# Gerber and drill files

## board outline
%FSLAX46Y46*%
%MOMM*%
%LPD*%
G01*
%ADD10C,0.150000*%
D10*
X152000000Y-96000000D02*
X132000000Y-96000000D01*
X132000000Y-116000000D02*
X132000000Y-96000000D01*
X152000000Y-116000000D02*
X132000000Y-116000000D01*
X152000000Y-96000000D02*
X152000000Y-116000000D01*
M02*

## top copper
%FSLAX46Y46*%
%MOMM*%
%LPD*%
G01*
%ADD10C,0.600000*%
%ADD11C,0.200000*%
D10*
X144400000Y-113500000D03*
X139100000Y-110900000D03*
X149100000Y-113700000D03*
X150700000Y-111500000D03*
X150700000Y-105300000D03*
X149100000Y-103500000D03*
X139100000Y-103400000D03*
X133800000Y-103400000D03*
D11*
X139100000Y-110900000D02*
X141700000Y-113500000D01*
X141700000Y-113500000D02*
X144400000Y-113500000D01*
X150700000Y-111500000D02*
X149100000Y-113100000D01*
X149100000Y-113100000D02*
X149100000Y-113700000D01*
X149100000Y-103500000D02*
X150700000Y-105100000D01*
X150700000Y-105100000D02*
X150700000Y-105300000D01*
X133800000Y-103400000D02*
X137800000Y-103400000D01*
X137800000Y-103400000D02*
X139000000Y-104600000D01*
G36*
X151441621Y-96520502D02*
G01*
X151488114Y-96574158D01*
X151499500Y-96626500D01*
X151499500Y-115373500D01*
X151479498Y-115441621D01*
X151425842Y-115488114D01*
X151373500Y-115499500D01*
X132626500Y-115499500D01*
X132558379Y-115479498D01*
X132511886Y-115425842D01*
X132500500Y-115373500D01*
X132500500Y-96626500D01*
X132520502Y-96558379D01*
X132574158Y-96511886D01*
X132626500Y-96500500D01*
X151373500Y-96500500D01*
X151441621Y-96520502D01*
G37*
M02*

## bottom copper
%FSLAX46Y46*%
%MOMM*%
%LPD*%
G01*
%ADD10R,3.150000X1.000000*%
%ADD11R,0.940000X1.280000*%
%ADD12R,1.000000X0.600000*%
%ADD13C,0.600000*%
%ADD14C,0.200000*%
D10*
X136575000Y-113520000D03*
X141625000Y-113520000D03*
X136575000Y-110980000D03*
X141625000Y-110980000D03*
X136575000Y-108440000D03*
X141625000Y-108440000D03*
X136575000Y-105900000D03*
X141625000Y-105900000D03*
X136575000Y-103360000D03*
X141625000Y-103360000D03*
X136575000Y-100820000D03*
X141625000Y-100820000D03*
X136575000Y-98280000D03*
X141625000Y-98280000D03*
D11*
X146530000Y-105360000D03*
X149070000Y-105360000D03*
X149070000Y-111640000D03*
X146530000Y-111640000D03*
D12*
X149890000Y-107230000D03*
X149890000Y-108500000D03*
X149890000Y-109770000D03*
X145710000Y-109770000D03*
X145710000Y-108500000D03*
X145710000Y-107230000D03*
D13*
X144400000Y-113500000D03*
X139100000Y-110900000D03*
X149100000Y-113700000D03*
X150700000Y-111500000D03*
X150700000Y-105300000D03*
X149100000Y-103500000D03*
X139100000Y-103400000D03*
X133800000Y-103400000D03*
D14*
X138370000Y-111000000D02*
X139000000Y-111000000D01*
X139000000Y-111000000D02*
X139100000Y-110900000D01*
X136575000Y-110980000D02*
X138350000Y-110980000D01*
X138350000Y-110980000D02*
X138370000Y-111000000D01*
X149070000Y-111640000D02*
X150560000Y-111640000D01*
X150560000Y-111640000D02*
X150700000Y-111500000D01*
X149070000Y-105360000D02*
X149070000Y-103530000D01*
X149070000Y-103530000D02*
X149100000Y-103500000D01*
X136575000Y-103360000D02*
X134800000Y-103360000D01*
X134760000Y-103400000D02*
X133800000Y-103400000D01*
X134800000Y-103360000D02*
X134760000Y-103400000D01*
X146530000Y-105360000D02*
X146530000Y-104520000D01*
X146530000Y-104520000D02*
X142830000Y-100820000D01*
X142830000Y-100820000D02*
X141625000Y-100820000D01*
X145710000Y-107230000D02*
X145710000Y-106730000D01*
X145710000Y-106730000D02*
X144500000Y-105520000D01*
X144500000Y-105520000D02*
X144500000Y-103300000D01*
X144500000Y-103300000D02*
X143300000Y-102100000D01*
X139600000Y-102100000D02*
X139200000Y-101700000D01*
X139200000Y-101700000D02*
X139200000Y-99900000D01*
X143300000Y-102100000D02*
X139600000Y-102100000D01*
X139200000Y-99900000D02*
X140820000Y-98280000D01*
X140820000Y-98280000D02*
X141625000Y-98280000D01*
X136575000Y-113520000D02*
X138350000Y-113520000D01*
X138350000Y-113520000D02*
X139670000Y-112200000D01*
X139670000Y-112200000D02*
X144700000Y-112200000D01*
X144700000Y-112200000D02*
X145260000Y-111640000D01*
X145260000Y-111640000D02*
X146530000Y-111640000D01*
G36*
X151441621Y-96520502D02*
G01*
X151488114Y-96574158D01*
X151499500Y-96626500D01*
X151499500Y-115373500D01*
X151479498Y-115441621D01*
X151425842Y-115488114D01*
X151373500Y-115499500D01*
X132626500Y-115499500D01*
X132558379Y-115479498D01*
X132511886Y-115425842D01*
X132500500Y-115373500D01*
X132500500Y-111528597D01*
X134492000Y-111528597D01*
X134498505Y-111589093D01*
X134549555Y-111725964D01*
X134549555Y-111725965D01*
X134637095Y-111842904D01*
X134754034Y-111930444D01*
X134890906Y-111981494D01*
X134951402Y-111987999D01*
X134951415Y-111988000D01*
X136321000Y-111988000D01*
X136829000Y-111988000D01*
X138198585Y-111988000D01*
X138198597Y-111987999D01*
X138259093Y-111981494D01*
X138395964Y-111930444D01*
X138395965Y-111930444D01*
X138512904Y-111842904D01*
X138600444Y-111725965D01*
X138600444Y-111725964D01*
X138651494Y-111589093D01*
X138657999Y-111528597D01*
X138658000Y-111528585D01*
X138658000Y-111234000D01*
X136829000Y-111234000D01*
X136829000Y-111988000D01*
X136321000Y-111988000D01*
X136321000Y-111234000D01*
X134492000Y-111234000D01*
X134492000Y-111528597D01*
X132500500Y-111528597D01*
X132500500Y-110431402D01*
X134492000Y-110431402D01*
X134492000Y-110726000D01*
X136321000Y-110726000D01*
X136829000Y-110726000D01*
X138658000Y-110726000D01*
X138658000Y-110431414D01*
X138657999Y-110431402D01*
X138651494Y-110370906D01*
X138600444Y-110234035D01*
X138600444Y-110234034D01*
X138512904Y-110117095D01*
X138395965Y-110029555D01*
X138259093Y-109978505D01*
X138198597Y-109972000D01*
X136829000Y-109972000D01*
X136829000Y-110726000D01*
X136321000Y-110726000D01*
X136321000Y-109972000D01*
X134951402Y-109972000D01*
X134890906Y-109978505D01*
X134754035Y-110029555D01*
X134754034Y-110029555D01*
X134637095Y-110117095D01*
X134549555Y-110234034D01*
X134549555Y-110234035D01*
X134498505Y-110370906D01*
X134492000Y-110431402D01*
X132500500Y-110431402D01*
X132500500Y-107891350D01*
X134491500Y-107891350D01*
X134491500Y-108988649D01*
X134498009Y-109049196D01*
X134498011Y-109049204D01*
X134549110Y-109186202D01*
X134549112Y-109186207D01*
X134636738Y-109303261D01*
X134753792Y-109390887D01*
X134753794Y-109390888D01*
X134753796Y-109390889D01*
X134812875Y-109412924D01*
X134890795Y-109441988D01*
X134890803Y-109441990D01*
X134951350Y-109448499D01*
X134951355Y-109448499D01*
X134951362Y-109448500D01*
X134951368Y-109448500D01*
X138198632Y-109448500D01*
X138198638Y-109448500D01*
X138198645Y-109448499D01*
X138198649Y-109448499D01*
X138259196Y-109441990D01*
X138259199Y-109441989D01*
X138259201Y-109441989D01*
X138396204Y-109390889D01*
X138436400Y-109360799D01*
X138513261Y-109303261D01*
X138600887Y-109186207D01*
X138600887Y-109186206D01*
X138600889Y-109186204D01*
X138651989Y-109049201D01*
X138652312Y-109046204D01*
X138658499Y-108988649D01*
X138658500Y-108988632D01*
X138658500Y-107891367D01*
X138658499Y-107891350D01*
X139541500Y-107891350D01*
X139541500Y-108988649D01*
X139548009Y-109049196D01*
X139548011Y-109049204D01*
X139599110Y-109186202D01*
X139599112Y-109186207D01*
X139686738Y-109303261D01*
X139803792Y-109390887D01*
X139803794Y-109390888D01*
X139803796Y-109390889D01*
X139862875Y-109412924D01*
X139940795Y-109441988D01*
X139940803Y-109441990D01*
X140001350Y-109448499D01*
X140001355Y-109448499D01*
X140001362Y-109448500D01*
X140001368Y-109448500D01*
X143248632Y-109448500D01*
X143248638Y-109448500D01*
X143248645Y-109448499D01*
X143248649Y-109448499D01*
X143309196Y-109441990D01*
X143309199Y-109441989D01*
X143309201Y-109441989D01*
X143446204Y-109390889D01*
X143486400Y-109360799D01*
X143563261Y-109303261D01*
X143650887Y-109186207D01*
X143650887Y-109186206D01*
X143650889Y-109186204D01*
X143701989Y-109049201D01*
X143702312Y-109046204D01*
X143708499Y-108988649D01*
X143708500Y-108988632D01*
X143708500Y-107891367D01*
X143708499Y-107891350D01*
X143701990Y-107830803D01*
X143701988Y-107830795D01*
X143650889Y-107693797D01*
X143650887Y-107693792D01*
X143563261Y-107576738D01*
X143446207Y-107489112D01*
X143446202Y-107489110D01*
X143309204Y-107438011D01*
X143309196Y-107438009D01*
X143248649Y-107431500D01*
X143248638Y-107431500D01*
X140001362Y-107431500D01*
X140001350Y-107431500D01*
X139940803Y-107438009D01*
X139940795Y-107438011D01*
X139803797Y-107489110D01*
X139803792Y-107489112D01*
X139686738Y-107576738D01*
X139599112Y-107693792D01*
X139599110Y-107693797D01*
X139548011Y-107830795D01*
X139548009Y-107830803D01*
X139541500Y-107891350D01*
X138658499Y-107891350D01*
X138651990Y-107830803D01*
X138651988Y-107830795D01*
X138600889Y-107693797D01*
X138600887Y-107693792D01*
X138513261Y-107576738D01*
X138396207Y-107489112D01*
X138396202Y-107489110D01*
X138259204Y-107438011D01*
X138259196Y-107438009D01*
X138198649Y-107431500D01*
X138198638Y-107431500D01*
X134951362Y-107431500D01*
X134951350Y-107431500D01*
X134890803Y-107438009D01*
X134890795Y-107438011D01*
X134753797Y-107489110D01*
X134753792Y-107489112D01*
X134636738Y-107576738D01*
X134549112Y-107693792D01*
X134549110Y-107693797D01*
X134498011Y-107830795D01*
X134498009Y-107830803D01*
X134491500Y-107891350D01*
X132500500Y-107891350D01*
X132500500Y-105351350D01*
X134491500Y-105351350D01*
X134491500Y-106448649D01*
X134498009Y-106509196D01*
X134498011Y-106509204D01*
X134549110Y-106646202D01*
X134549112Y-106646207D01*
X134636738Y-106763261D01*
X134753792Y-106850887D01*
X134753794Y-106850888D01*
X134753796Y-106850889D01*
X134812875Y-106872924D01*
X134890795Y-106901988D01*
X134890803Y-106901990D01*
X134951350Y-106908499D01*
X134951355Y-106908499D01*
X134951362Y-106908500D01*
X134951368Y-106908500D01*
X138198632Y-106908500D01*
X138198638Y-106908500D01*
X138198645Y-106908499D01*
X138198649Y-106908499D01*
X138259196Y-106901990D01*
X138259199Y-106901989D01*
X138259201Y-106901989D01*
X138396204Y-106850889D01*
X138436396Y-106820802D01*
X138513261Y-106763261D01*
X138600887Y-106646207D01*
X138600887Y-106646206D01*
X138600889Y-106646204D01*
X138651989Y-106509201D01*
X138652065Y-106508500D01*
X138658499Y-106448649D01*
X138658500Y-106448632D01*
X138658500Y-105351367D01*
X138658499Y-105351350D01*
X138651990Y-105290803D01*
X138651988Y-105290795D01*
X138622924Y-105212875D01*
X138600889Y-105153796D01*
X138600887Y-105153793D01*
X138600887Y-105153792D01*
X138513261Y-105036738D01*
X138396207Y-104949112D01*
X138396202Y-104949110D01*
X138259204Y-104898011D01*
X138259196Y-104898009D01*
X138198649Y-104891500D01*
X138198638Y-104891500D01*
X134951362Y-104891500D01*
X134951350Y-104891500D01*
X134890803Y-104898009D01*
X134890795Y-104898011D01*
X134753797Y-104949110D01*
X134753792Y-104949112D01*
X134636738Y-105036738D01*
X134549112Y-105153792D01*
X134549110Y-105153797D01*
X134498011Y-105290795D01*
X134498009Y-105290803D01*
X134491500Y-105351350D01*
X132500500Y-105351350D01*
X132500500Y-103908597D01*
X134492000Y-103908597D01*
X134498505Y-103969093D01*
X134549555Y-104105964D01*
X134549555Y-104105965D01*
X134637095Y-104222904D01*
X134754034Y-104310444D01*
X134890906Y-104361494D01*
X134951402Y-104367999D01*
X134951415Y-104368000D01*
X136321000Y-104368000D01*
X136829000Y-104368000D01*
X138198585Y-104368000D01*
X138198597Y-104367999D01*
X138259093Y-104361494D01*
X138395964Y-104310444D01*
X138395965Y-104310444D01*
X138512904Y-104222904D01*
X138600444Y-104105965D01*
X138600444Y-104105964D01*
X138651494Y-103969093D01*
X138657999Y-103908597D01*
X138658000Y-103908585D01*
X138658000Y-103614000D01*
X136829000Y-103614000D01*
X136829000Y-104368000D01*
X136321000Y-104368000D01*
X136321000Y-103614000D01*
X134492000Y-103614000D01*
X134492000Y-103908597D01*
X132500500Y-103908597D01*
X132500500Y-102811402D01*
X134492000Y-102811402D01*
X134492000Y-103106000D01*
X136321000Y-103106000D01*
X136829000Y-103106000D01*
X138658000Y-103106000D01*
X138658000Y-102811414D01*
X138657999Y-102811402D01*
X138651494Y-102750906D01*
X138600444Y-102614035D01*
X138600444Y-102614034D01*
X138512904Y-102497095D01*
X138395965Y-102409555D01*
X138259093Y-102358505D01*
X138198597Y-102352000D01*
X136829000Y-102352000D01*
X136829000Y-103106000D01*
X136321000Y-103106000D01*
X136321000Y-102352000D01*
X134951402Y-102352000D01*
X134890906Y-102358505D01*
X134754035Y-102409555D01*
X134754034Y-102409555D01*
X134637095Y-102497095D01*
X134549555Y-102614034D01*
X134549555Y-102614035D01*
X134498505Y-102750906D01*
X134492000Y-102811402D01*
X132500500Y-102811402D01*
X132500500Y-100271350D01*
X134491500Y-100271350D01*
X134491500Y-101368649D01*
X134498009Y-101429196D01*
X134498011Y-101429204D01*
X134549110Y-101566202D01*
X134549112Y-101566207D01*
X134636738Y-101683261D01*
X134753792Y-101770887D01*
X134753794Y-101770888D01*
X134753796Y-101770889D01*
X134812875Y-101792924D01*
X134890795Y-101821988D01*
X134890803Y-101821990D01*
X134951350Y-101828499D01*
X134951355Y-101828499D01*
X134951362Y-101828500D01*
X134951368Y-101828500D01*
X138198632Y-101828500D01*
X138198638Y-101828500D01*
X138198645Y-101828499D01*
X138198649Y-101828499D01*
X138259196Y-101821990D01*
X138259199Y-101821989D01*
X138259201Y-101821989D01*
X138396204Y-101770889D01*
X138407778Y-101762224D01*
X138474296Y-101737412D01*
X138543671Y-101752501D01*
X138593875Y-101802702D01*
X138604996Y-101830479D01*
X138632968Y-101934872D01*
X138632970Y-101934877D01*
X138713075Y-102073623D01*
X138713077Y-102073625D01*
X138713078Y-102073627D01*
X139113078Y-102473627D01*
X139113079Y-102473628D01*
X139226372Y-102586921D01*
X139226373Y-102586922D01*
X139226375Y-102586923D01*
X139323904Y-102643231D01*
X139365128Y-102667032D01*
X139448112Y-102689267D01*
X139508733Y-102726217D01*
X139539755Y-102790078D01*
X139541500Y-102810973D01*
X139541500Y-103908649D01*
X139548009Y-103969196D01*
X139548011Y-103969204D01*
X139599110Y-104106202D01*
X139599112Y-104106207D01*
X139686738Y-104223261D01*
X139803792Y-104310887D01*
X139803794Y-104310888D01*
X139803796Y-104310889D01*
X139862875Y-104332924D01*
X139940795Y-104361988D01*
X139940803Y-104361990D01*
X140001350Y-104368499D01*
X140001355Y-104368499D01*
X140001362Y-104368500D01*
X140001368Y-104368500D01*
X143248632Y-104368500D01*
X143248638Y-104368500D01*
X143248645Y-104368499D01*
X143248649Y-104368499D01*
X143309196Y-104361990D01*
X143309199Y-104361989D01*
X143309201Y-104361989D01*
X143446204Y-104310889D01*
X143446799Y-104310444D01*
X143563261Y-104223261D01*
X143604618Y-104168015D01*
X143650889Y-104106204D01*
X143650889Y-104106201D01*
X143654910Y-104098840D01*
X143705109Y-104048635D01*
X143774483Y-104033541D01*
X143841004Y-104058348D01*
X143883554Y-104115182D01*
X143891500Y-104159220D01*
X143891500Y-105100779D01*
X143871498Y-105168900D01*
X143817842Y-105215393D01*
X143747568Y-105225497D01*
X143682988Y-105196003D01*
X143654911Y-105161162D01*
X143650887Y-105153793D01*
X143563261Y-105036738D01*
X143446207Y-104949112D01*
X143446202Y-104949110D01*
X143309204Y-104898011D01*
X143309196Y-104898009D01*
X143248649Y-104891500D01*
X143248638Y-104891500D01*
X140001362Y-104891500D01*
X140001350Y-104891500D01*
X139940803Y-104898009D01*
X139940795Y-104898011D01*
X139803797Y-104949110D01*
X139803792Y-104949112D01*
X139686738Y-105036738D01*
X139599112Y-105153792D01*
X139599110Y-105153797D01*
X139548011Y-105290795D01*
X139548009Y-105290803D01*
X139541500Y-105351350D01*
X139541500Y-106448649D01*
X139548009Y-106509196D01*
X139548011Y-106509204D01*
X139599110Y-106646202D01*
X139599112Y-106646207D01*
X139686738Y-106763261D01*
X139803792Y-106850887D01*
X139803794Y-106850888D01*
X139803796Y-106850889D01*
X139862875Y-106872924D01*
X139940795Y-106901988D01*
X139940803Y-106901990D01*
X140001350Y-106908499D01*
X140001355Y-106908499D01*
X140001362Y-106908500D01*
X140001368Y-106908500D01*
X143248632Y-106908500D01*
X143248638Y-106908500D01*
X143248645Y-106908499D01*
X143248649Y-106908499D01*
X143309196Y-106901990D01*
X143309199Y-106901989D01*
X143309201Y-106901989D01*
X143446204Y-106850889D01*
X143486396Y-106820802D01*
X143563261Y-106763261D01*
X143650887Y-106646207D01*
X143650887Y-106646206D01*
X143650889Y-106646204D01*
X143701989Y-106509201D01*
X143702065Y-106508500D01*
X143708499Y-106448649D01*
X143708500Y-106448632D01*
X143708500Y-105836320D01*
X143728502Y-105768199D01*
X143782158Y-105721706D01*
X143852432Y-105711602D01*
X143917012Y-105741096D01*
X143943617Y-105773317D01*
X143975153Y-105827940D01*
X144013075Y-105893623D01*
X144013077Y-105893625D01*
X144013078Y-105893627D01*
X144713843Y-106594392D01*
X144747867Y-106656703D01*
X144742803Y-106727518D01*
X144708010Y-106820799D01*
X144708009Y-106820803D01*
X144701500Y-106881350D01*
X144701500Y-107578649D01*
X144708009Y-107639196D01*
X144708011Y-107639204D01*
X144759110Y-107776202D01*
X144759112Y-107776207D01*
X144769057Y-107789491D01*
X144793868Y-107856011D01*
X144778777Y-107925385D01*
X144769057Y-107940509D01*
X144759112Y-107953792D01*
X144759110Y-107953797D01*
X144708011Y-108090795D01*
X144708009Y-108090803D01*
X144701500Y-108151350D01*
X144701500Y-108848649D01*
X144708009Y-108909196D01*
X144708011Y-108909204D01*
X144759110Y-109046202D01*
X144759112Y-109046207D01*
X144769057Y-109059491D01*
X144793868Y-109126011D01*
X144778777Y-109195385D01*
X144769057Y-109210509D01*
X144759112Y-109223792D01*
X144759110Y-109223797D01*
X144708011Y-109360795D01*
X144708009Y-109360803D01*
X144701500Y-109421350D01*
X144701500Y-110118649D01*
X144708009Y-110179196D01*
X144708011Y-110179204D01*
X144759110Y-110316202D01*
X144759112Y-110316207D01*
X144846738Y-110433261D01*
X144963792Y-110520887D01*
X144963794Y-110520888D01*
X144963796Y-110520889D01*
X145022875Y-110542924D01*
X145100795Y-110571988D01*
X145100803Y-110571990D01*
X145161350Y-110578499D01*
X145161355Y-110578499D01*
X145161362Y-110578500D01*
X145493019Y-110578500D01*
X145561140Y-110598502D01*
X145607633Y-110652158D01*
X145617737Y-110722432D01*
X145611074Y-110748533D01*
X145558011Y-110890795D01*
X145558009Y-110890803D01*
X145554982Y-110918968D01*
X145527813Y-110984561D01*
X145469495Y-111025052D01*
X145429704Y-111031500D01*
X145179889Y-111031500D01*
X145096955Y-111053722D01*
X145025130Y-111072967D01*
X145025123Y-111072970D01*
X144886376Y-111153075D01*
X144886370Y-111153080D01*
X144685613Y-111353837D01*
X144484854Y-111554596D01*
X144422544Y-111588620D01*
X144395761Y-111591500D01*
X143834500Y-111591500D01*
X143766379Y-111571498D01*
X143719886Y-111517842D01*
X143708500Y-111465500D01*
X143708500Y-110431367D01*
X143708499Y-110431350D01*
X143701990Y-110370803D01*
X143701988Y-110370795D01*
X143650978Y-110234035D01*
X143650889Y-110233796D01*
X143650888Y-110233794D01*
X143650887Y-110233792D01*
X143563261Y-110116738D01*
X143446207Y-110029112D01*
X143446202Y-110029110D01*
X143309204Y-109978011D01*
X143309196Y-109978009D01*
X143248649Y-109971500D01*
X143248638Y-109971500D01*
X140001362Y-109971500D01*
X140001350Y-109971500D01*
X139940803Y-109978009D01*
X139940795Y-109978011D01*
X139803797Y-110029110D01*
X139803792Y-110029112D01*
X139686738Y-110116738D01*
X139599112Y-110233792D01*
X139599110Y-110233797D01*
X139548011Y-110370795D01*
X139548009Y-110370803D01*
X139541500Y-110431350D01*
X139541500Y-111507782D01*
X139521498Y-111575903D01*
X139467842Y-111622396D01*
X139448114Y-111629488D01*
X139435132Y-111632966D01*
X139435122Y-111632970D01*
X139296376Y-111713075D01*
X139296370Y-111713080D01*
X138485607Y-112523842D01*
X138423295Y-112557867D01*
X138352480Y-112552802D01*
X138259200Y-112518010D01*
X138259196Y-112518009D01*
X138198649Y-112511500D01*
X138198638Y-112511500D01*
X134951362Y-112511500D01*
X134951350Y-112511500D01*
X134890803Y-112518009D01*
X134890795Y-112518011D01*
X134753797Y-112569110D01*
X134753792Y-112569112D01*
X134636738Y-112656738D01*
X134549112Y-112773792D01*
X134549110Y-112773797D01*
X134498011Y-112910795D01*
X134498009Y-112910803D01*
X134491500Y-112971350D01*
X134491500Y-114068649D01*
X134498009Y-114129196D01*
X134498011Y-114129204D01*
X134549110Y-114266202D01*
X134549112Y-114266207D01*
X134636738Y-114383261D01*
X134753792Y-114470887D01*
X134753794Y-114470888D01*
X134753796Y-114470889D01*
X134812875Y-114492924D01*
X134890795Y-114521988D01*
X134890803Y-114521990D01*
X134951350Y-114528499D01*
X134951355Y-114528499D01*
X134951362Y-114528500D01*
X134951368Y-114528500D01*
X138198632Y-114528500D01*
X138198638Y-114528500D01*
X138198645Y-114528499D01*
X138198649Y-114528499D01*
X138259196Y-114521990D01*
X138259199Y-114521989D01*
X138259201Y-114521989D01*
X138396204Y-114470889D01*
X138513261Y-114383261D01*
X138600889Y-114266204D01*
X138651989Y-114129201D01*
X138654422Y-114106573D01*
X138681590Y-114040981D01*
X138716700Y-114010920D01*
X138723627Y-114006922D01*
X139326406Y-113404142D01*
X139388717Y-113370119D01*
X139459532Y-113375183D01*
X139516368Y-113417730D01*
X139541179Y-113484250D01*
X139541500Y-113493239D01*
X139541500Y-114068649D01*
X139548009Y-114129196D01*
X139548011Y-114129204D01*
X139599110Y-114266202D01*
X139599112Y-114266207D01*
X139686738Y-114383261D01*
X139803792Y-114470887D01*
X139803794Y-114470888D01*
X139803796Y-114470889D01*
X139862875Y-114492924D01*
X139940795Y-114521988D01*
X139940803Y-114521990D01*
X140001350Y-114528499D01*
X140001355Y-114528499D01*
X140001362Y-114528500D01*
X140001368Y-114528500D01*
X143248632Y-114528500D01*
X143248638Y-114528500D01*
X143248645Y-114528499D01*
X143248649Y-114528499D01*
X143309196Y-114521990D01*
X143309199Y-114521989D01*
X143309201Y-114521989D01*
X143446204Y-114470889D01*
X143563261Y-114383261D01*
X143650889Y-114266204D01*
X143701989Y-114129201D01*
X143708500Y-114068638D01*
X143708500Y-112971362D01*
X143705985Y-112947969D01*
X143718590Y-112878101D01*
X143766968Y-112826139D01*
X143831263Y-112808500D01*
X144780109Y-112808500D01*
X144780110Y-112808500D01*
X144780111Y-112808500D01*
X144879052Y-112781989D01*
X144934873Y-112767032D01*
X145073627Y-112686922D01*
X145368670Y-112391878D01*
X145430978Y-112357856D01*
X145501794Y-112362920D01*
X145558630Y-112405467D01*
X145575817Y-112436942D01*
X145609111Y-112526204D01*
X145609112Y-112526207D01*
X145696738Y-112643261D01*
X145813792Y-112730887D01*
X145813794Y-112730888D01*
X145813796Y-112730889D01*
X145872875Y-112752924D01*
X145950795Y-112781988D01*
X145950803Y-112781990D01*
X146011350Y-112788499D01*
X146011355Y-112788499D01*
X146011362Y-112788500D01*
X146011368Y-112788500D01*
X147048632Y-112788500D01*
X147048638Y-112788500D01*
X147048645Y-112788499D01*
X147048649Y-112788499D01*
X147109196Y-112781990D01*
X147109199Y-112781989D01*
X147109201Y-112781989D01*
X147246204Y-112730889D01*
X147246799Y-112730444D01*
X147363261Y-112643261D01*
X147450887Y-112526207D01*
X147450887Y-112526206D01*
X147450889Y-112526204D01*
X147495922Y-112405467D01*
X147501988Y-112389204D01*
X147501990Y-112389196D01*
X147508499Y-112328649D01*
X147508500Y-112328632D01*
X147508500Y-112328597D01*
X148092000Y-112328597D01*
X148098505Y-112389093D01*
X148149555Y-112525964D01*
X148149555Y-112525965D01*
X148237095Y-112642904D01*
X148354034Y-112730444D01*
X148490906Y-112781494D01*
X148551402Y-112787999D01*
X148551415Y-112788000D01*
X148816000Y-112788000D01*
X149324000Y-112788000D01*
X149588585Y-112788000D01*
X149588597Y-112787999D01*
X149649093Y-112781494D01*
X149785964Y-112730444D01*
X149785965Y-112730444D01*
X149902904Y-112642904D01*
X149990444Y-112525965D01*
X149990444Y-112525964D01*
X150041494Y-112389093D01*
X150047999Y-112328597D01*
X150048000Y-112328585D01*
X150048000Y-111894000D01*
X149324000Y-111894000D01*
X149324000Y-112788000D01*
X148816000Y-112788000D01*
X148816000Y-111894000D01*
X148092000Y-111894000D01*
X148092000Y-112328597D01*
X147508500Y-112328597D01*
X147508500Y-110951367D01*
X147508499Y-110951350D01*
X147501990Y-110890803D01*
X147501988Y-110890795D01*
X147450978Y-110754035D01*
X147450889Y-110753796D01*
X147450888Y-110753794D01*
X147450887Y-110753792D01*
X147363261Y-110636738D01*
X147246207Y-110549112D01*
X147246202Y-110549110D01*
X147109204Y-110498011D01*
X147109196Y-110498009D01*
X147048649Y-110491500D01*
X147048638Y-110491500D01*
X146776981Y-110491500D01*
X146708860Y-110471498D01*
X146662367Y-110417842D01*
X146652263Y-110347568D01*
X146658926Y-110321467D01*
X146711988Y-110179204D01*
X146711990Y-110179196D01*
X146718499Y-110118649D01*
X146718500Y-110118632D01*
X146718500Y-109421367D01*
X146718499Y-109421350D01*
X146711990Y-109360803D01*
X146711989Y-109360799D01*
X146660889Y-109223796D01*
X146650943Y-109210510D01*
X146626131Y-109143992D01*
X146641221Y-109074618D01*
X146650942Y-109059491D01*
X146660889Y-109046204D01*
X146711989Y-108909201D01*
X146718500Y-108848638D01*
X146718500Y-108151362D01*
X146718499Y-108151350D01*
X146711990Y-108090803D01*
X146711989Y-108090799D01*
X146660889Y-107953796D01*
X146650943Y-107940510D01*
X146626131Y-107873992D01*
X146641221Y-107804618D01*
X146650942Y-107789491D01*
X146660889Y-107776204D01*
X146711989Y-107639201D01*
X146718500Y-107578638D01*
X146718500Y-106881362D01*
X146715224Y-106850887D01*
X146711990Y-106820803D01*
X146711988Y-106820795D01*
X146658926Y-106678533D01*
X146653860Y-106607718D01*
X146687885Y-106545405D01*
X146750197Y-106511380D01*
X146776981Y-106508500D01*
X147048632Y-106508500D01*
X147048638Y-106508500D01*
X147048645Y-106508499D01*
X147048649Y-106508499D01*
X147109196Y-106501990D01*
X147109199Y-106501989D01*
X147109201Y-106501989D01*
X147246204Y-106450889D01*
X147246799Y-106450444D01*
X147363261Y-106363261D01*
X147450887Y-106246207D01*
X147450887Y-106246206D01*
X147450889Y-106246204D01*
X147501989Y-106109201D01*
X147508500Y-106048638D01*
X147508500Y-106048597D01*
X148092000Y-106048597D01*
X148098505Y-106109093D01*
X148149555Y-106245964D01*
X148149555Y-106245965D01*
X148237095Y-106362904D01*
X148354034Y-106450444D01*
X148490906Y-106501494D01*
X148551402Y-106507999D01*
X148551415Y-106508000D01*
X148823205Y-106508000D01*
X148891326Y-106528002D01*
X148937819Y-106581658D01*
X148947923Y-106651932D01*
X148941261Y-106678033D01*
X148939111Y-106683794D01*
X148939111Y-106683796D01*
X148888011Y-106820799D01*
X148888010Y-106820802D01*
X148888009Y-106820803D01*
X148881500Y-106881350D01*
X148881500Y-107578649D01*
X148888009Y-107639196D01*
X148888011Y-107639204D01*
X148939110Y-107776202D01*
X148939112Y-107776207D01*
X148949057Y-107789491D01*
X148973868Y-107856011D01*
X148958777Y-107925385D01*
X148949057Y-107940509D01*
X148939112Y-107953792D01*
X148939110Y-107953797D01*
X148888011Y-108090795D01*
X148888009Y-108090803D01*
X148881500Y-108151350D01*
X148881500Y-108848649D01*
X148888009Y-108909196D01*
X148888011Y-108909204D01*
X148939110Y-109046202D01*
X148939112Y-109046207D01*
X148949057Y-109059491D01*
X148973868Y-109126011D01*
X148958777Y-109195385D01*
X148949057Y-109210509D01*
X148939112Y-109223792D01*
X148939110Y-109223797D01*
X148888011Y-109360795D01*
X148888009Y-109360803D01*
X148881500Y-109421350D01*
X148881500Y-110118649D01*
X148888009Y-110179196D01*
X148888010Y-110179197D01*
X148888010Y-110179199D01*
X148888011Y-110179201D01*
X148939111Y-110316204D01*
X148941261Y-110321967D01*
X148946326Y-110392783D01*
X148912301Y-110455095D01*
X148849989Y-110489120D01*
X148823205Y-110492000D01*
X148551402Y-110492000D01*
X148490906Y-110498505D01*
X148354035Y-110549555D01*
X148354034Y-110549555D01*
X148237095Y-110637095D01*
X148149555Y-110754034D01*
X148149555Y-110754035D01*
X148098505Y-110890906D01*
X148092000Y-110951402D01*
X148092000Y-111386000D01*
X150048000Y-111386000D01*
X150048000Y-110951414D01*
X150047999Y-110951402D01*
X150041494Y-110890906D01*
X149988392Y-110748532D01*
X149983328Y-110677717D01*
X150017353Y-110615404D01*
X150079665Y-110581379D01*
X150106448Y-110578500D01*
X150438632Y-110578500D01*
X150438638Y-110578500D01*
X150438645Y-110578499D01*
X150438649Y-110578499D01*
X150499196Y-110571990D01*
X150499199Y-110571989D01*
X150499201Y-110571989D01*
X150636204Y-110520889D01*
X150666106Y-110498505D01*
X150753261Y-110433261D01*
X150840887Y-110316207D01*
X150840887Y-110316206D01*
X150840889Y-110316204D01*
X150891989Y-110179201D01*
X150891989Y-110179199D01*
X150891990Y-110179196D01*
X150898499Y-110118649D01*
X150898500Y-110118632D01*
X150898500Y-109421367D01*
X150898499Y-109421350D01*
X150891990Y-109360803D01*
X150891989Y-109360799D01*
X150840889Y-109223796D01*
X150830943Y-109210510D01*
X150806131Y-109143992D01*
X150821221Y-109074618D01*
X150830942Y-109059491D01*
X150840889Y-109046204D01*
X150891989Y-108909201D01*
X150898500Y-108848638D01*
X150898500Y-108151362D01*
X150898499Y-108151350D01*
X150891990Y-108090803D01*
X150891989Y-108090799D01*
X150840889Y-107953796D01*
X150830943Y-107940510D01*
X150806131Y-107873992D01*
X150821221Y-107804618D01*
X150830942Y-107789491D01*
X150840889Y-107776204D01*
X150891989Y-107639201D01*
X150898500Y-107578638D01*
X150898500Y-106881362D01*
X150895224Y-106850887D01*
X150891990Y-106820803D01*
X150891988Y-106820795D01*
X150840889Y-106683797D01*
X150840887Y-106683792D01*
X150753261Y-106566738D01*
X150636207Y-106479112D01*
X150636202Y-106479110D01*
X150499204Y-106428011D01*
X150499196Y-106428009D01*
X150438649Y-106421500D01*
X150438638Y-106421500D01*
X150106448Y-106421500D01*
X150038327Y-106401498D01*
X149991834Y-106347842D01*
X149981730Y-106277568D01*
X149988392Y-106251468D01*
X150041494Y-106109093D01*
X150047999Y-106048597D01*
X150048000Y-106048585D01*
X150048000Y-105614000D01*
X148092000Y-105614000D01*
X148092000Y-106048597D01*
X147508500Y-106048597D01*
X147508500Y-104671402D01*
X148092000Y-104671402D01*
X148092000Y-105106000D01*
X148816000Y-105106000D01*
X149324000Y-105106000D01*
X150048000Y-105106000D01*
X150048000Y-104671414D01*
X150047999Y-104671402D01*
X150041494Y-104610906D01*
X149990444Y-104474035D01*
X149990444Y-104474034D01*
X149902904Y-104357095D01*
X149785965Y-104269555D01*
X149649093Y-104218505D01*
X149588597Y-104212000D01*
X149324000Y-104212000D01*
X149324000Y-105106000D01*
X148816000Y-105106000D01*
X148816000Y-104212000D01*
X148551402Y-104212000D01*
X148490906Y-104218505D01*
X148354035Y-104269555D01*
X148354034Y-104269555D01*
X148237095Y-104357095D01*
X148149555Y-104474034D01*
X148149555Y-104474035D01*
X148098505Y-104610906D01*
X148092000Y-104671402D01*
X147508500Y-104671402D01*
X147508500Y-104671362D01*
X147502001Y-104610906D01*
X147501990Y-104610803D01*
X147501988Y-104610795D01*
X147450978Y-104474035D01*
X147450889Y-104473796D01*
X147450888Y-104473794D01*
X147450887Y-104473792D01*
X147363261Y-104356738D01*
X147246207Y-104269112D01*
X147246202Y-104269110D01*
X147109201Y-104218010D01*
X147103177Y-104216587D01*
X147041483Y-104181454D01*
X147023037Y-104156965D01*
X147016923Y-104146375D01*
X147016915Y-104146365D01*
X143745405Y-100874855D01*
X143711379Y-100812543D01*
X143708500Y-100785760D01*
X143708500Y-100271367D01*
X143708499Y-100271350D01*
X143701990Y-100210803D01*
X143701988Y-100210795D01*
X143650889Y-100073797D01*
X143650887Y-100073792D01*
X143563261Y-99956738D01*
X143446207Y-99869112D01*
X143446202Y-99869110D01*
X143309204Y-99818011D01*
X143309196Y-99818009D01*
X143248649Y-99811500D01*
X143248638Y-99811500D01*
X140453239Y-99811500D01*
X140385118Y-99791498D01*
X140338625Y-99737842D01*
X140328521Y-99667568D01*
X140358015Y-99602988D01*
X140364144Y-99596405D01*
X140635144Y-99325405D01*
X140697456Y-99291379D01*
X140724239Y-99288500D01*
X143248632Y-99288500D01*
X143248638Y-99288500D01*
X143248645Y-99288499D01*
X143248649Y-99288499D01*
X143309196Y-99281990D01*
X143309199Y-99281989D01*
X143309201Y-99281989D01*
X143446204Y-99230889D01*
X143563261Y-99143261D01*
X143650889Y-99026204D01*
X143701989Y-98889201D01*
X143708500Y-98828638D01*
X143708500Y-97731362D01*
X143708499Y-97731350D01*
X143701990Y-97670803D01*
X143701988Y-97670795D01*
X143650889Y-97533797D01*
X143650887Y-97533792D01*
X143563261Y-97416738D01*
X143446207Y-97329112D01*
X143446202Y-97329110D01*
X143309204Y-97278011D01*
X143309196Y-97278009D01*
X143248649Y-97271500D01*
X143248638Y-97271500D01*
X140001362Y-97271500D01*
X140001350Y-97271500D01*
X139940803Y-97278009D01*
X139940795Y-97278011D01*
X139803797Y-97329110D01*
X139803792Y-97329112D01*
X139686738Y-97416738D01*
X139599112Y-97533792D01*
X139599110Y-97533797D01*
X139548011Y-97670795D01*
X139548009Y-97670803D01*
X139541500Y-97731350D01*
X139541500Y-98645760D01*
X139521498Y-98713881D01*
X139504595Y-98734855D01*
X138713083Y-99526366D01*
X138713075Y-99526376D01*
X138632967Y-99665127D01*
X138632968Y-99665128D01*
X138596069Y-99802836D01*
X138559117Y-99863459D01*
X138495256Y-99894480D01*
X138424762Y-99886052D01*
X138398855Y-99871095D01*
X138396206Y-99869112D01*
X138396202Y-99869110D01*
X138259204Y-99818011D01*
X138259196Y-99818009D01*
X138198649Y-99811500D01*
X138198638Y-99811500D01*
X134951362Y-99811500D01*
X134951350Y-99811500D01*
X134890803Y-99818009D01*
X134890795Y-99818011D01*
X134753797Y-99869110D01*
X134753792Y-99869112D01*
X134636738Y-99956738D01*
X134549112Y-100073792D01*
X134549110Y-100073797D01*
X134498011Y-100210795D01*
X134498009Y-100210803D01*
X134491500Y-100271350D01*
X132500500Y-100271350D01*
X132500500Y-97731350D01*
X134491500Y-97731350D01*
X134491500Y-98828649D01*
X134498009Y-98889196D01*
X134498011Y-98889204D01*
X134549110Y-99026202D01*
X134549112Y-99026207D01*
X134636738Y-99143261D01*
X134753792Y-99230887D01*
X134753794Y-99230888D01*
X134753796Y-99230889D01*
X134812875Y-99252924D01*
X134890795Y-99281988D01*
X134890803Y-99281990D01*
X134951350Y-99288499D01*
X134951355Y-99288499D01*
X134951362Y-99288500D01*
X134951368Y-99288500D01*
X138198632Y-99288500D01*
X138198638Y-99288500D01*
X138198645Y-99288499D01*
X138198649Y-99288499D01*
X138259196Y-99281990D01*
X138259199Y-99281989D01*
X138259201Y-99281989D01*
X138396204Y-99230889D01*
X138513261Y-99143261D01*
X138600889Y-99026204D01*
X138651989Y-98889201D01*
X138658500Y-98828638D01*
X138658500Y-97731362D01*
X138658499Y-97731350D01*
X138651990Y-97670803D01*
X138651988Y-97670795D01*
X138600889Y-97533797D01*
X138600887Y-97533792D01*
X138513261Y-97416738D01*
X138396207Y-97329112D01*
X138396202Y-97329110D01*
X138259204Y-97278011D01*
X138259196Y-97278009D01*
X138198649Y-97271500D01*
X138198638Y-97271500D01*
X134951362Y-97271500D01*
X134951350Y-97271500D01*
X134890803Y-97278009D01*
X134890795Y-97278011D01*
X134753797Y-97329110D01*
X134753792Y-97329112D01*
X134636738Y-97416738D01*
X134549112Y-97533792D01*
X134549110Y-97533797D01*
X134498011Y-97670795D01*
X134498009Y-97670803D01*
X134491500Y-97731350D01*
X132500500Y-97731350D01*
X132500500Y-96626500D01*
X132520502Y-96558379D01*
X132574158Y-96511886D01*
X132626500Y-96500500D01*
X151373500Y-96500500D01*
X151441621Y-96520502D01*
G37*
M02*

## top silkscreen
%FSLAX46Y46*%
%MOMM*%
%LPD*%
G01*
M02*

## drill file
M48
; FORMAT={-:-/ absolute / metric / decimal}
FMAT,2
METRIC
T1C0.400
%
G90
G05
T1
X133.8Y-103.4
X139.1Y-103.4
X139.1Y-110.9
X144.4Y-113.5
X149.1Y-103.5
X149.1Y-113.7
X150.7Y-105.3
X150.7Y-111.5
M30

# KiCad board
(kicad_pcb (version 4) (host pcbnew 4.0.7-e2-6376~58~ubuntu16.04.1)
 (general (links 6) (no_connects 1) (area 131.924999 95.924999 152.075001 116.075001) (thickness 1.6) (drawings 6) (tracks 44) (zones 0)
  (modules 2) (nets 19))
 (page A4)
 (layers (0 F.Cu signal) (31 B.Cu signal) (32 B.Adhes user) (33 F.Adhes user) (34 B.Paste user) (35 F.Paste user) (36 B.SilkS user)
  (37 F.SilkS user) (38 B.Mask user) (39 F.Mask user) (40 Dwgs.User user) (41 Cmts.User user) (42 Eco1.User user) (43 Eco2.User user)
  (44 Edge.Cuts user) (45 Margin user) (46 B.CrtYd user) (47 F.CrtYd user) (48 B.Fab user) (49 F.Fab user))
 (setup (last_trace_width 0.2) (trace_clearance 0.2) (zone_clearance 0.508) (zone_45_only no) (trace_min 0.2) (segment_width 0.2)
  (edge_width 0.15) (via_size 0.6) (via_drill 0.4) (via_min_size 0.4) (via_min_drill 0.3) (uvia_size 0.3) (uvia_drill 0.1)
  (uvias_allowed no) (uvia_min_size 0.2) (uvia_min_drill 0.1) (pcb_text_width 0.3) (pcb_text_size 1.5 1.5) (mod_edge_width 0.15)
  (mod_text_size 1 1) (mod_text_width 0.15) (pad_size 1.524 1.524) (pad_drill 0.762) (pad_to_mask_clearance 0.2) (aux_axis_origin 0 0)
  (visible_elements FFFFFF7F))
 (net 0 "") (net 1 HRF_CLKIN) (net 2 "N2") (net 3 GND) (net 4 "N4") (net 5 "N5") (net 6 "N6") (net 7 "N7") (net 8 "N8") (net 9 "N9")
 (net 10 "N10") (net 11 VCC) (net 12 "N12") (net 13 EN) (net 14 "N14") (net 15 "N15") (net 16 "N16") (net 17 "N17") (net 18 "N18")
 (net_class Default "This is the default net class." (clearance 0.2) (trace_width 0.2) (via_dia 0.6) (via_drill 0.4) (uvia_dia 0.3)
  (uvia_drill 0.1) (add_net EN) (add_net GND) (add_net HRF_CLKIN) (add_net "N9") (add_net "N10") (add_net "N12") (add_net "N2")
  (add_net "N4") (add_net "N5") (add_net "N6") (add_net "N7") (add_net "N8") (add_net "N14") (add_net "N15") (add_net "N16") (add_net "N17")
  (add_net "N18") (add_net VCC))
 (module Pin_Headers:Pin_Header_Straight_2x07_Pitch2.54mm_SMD (layer B.Cu) (at 139.1 105.9)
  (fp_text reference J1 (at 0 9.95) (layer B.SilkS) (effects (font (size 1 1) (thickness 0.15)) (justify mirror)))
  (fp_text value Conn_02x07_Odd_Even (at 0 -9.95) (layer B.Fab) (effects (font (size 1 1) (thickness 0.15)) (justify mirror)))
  (pad 1 smd rect (at -2.525 7.62) (size 3.15 1) (layers B.Cu B.Paste B.Mask) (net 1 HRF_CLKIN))
  (pad 2 smd rect (at 2.525 7.62) (size 3.15 1) (layers B.Cu B.Paste B.Mask) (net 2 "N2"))
  (pad 3 smd rect (at -2.525 5.08) (size 3.15 1) (layers B.Cu B.Paste B.Mask) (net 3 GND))
  (pad 4 smd rect (at 2.525 5.08) (size 3.15 1) (layers B.Cu B.Paste B.Mask) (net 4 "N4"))
  (pad 5 smd rect (at -2.525 2.54) (size 3.15 1) (layers B.Cu B.Paste B.Mask) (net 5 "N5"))
  (pad 6 smd rect (at 2.525 2.54) (size 3.15 1) (layers B.Cu B.Paste B.Mask) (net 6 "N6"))
  (pad 7 smd rect (at -2.525 0) (size 3.15 1) (layers B.Cu B.Paste B.Mask) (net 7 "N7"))
  (pad 8 smd rect (at 2.525 0) (size 3.15 1) (layers B.Cu B.Paste B.Mask) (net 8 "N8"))
  (pad 9 smd rect (at -2.525 -2.54) (size 3.15 1) (layers B.Cu B.Paste B.Mask) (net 3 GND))
  (pad 10 smd rect (at 2.525 -2.54) (size 3.15 1) (layers B.Cu B.Paste B.Mask) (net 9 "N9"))
  (pad 11 smd rect (at -2.525 -5.08) (size 3.15 1) (layers B.Cu B.Paste B.Mask) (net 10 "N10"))
  (pad 12 smd rect (at 2.525 -5.08) (size 3.15 1) (layers B.Cu B.Paste B.Mask) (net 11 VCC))
  (pad 13 smd rect (at -2.525 -7.62) (size 3.15 1) (layers B.Cu B.Paste B.Mask) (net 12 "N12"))
  (pad 14 smd rect (at 2.525 -7.62) (size 3.15 1) (layers B.Cu B.Paste B.Mask) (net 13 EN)))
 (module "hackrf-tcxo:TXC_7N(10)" (layer B.Cu) (at 147.8 108.5 270)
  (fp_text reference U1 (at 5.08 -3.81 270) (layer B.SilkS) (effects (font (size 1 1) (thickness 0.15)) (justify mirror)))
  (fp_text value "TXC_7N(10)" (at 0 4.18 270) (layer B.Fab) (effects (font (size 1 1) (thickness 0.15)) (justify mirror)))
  (pad 9 smd rect (at -3.14 1.27 270) (size 1.28 0.94) (layers B.Cu B.Paste B.Mask) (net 11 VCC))
  (pad 10 smd rect (at -3.14 -1.27 270) (size 1.28 0.94) (layers B.Cu B.Paste B.Mask) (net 3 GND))
  (pad 4 smd rect (at 3.14 -1.27 270) (size 1.28 0.94) (layers B.Cu B.Paste B.Mask) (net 3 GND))
  (pad 5 smd rect (at 3.14 1.27 270) (size 1.28 0.94) (layers B.Cu B.Paste B.Mask) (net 1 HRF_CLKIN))
  (pad 1 smd rect (at -1.27 -2.09 270) (size 0.6 1) (layers B.Cu B.Paste B.Mask) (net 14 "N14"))
  (pad 2 smd rect (at 0 -2.09 270) (size 0.6 1) (layers B.Cu B.Paste B.Mask) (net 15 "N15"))
  (pad 3 smd rect (at 1.27 -2.09 270) (size 0.6 1) (layers B.Cu B.Paste B.Mask) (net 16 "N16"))
  (pad 6 smd rect (at 1.27 2.09 270) (size 0.6 1) (layers B.Cu B.Paste B.Mask) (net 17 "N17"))
  (pad 7 smd rect (at 0 2.09 270) (size 0.6 1) (layers B.Cu B.Paste B.Mask) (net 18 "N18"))
  (pad 8 smd rect (at -1.27 2.09 270) (size 0.6 1) (layers B.Cu B.Paste B.Mask) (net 13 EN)))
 (gr_line (start 152 96) (end 132 96) (angle 90) (layer Edge.Cuts) (width 0.15))
 (gr_line (start 132 116) (end 132 96) (angle 90) (layer Edge.Cuts) (width 0.15))
 (gr_line (start 152 116) (end 132 116) (angle 90) (layer Edge.Cuts) (width 0.15))
 (gr_line (start 152 96) (end 152 116) (angle 90) (layer Edge.Cuts) (width 0.15))
 (segment (start 139.1 110.9) (end 141.7 113.5) (width 0.2) (layer F.Cu) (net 3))
 (segment (start 141.7 113.5) (end 144.4 113.5) (width 0.2) (layer F.Cu) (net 3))
 (via (at 144.4 113.5) (size 0.6) (drill 0.4) (layers F.Cu B.Cu) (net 3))
 (segment (start 138.37 111) (end 139 111) (width 0.2) (layer B.Cu) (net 3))
 (segment (start 139 111) (end 139.1 110.9) (width 0.2) (layer B.Cu) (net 3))
 (via (at 139.1 110.9) (size 0.6) (drill 0.4) (layers F.Cu B.Cu) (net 3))
 (segment (start 136.575 110.98) (end 138.35 110.98) (width 0.2) (layer B.Cu) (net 3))
 (segment (start 138.35 110.98) (end 138.37 111) (width 0.2) (layer B.Cu) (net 3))
 (segment (start 150.7 111.5) (end 149.1 113.1) (width 0.2) (layer F.Cu) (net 3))
 (segment (start 149.1 113.1) (end 149.1 113.7) (width 0.2) (layer F.Cu) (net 3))
 (via (at 149.1 113.7) (size 0.6) (drill 0.4) (layers F.Cu B.Cu) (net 3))
 (segment (start 149.07 111.64) (end 150.56 111.64) (width 0.2) (layer B.Cu) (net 3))
 (segment (start 150.56 111.64) (end 150.7 111.5) (width 0.2) (layer B.Cu) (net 3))
 (via (at 150.7 111.5) (size 0.6) (drill 0.4) (layers F.Cu B.Cu) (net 3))
 (segment (start 149.1 103.5) (end 150.7 105.1) (width 0.2) (layer F.Cu) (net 3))
 (via (at 150.7 105.3) (size 0.6) (drill 0.4) (layers F.Cu B.Cu) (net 3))
 (segment (start 150.7 105.1) (end 150.7 105.3) (width 0.2) (layer F.Cu) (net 3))
 (segment (start 149.07 105.36) (end 149.07 103.53) (width 0.2) (layer B.Cu) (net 3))
 (via (at 149.1 103.5) (size 0.6) (drill 0.4) (layers F.Cu B.Cu) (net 3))
 (segment (start 149.07 103.53) (end 149.1 103.5) (width 0.2) (layer B.Cu) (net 3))
 (segment (start 133.8 103.4) (end 137.8 103.4) (width 0.2) (layer F.Cu) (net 3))
 (segment (start 137.8 103.4) (end 139 104.6) (width 0.2) (layer F.Cu) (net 3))
 (via (at 139.1 103.4) (size 0.6) (drill 0.4) (layers F.Cu B.Cu) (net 3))
 (segment (start 136.575 103.36) (end 134.8 103.36) (width 0.2) (layer B.Cu) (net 3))
 (segment (start 134.76 103.4) (end 133.8 103.4) (width 0.2) (layer B.Cu) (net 3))
 (segment (start 134.8 103.36) (end 134.76 103.4) (width 0.2) (layer B.Cu) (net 3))
 (via (at 133.8 103.4) (size 0.6) (drill 0.4) (layers F.Cu B.Cu) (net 3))
 (segment (start 146.53 105.36) (end 146.53 104.52) (width 0.2) (layer B.Cu) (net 11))
 (segment (start 146.53 104.52) (end 142.83 100.82) (width 0.2) (layer B.Cu) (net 11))
 (segment (start 142.83 100.82) (end 141.625 100.82) (width 0.2) (layer B.Cu) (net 11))
 (segment (start 145.71 107.23) (end 145.71 106.73) (width 0.2) (layer B.Cu) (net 13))
 (segment (start 145.71 106.73) (end 144.5 105.52) (width 0.2) (layer B.Cu) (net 13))
 (segment (start 144.5 105.52) (end 144.5 103.3) (width 0.2) (layer B.Cu) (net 13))
 (segment (start 144.5 103.3) (end 143.3 102.1) (width 0.2) (layer B.Cu) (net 13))
 (segment (start 139.6 102.1) (end 139.2 101.7) (width 0.2) (layer B.Cu) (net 13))
 (segment (start 139.2 101.7) (end 139.2 99.9) (width 0.2) (layer B.Cu) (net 13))
 (segment (start 143.3 102.1) (end 139.6 102.1) (width 0.2) (layer B.Cu) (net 13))
 (segment (start 139.2 99.9) (end 140.82 98.28) (width 0.2) (layer B.Cu) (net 13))
 (segment (start 140.82 98.28) (end 141.625 98.28) (width 0.2) (layer B.Cu) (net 13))
 (segment (start 136.575 113.52) (end 138.35 113.52) (width 0.2) (layer B.Cu) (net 1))
 (segment (start 138.35 113.52) (end 139.67 112.2) (width 0.2) (layer B.Cu) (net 1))
 (segment (start 139.67 112.2) (end 144.7 112.2) (width 0.2) (layer B.Cu) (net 1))
 (segment (start 144.7 112.2) (end 145.26 111.64) (width 0.2) (layer B.Cu) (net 1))
 (segment (start 145.26 111.64) (end 146.53 111.64) (width 0.2) (layer B.Cu) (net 1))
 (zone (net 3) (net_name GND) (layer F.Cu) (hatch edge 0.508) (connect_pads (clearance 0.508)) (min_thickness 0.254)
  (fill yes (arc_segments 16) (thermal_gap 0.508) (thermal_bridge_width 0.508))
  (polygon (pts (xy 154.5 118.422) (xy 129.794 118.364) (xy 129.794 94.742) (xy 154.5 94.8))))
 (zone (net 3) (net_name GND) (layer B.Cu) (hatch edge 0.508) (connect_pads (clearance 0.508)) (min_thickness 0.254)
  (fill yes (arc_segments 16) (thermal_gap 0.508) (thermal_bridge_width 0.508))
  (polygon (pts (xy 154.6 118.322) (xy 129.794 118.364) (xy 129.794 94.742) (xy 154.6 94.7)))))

